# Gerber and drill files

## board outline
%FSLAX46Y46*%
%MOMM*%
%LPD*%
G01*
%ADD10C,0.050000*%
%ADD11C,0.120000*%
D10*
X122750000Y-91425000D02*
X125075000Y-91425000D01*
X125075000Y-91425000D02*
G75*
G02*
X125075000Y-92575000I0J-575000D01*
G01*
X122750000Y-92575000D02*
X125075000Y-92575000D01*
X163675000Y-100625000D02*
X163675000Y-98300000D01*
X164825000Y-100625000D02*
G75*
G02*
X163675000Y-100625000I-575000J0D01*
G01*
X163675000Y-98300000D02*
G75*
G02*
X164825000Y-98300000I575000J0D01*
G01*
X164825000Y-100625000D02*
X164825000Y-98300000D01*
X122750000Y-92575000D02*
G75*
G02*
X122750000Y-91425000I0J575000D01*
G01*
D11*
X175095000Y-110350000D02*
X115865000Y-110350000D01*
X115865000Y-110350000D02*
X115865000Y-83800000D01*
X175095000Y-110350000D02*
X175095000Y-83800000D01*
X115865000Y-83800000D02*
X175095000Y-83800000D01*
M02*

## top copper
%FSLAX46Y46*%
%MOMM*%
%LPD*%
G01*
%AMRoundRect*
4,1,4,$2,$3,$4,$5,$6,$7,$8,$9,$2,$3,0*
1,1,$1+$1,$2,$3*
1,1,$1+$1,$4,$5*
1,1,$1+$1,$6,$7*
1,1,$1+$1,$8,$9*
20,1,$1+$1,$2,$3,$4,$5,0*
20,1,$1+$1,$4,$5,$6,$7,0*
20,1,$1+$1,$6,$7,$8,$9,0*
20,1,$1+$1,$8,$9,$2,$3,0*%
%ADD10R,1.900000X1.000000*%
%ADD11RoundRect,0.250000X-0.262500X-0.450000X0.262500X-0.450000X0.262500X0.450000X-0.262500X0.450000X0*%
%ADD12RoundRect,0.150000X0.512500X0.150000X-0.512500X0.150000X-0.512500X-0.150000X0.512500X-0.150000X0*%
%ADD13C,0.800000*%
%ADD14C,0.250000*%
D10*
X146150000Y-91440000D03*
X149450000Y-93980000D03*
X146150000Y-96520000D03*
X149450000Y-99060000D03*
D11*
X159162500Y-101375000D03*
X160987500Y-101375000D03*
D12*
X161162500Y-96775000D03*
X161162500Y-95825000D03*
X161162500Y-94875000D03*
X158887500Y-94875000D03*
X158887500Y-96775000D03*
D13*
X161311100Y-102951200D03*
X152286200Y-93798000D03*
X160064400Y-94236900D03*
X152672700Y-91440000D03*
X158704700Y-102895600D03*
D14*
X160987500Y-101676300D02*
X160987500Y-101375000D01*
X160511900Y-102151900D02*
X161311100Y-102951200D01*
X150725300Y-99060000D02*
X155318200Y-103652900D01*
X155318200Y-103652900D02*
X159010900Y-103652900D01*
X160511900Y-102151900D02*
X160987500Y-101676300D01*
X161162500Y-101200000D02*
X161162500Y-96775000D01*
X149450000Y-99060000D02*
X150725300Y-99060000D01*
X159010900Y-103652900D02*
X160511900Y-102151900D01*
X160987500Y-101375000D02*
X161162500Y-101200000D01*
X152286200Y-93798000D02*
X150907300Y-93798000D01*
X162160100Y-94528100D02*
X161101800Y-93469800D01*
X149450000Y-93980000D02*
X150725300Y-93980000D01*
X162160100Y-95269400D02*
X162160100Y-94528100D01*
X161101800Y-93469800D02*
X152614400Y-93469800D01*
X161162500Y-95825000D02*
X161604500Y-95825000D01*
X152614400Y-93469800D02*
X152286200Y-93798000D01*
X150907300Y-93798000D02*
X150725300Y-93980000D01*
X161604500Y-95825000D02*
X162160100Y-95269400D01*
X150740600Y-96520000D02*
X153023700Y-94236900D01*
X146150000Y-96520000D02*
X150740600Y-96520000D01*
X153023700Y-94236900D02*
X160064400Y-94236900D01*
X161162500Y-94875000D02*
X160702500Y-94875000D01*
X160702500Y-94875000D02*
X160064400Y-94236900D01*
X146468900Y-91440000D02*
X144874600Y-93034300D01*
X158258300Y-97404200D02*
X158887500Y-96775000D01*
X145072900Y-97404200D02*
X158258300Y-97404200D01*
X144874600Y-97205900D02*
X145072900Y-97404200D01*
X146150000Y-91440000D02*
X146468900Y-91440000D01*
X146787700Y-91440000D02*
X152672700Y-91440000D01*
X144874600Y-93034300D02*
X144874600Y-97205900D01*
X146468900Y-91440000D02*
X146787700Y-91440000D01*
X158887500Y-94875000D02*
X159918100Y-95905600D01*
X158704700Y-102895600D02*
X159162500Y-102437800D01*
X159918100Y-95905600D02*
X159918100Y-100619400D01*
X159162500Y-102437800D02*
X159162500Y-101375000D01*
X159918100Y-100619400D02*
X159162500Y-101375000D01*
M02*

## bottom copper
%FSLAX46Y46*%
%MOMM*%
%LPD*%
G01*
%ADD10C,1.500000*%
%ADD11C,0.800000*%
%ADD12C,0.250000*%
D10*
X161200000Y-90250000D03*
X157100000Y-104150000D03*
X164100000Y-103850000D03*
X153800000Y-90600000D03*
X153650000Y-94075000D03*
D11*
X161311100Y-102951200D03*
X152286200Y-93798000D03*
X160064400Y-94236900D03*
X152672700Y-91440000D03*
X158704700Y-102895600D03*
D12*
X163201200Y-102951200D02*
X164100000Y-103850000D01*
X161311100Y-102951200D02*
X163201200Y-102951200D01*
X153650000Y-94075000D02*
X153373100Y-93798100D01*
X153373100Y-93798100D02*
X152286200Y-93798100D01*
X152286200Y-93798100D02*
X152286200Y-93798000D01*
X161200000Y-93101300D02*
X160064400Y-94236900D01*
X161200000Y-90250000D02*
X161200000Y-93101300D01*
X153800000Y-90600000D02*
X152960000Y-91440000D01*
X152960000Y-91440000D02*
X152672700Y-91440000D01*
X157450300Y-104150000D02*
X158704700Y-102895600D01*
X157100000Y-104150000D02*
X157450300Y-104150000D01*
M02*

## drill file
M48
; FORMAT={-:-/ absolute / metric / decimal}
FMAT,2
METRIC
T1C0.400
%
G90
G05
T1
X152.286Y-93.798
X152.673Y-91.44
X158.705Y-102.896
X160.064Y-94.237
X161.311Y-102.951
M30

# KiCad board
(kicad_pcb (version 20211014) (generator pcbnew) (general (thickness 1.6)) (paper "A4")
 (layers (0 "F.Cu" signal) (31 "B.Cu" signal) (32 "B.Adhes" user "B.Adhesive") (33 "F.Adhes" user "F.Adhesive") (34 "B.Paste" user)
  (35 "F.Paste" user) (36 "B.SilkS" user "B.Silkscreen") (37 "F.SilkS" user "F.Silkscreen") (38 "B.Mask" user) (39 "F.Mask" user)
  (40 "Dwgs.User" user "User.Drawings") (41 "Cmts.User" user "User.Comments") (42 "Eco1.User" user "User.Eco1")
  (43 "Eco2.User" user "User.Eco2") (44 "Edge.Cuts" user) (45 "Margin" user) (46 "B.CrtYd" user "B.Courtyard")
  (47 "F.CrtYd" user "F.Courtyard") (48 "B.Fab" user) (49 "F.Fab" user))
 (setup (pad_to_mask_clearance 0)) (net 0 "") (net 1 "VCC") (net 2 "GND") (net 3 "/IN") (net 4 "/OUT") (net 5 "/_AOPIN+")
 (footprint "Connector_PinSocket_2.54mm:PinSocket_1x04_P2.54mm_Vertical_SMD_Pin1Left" (layer "F.Cu") (at 147.8 95.25)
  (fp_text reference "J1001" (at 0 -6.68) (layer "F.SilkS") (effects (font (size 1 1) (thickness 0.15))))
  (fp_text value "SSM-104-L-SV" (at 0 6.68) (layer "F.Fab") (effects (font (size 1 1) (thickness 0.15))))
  (pad "1" smd rect locked (at -1.65 -3.81) (size 1.9 1) (layers "F.Cu" "F.Paste" "F.Mask") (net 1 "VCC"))
  (pad "2" smd rect locked (at 1.65 -1.27) (size 1.9 1) (layers "F.Cu" "F.Paste" "F.Mask") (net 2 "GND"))
  (pad "3" smd rect locked (at -1.65 1.27) (size 1.9 1) (layers "F.Cu" "F.Paste" "F.Mask") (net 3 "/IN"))
  (pad "4" smd rect locked (at 1.65 3.81) (size 1.9 1) (layers "F.Cu" "F.Paste" "F.Mask") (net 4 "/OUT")))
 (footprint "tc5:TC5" (layer "F.Cu") (at 135.3 97.9)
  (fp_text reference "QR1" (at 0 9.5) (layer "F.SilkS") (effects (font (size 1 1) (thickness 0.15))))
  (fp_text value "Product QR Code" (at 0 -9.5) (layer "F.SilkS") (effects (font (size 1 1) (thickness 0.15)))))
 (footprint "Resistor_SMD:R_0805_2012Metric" (layer "F.Cu") (at 160.075 101.375)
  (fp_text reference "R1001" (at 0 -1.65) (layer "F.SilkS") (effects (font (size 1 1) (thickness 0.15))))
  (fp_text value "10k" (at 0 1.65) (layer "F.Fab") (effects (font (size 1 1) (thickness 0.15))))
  (pad "1" smd roundrect locked (at -0.9125 0) (size 1.025 1.4) (layers "F.Cu" "F.Paste" "F.Mask") (roundrect_rratio 0.243902)
   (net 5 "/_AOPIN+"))
  (pad "2" smd roundrect locked (at 0.9125 0) (size 1.025 1.4) (layers "F.Cu" "F.Paste" "F.Mask") (roundrect_rratio 0.243902) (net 4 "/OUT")))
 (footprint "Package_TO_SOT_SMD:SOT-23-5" (layer "F.Cu") (at 160.025 95.825 180)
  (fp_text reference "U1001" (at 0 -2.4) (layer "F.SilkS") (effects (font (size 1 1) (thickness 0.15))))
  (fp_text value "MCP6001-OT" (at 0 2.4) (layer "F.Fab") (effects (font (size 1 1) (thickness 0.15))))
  (pad "1" smd roundrect locked (at -1.1375 -0.95 180) (size 1.325 0.6) (layers "F.Cu" "F.Paste" "F.Mask") (roundrect_rratio 0.25)
   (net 4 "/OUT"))
  (pad "2" smd roundrect locked (at -1.1375 0 180) (size 1.325 0.6) (layers "F.Cu" "F.Paste" "F.Mask") (roundrect_rratio 0.25) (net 2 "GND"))
  (pad "3" smd roundrect locked (at -1.1375 0.95 180) (size 1.325 0.6) (layers "F.Cu" "F.Paste" "F.Mask") (roundrect_rratio 0.25)
   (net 3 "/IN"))
  (pad "4" smd roundrect locked (at 1.1375 0.95 180) (size 1.325 0.6) (layers "F.Cu" "F.Paste" "F.Mask") (roundrect_rratio 0.25)
   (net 5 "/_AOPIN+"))
  (pad "5" smd roundrect locked (at 1.1375 -0.95 180) (size 1.325 0.6) (layers "F.Cu" "F.Paste" "F.Mask") (roundrect_rratio 0.25)
   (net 1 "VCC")))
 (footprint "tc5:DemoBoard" (layer "F.Cu") (at 127.325 91.1)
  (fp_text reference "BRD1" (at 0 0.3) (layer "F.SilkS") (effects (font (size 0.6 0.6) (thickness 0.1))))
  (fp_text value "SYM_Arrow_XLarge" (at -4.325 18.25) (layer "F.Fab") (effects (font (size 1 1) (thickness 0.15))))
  (fp_line (start 47.77 19.25) (end -11.46 19.25) (layer "Edge.Cuts") (width 0.12))
  (fp_line (start -11.46 19.25) (end -11.46 -7.3) (layer "Edge.Cuts") (width 0.12))
  (fp_line (start 47.77 19.25) (end 47.77 -7.3) (layer "Edge.Cuts") (width 0.12))
  (fp_line (start -11.46 -7.3) (end 47.77 -7.3) (layer "Edge.Cuts") (width 0.12)))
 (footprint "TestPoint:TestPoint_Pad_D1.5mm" (layer "B.Cu") (at 161.2 90.25)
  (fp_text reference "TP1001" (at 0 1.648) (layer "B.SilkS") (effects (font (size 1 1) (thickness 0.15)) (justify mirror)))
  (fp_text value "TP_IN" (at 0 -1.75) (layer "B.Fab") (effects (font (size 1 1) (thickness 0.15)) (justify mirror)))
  (pad "1" smd circle locked (at 0 0) (size 1.5 1.5) (layers "B.Cu" "B.Mask") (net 3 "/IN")))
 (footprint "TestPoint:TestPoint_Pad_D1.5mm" (layer "B.Cu") (at 157.1 104.15)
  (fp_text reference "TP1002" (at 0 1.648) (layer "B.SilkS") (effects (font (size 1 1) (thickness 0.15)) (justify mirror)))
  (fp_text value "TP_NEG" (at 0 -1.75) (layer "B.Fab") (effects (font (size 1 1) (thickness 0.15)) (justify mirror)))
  (pad "1" smd circle locked (at 0 0) (size 1.5 1.5) (layers "B.Cu" "B.Mask") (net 5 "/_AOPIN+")))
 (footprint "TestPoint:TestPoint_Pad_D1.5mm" (layer "B.Cu") (at 164.1 103.85 180)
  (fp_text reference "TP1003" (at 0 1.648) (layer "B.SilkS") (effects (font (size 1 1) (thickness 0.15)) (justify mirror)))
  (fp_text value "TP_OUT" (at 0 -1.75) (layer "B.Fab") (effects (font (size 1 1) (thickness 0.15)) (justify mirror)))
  (pad "1" smd circle locked (at 0 0 180) (size 1.5 1.5) (layers "B.Cu" "B.Mask") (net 4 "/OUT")))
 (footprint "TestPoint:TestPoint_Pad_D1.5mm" (layer "B.Cu") (at 153.8 90.6)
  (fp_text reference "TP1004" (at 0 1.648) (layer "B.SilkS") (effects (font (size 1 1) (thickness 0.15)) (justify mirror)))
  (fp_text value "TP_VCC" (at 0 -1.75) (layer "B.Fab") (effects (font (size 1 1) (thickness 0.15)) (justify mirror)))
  (pad "1" smd circle locked (at 0 0) (size 1.5 1.5) (layers "B.Cu" "B.Mask") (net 1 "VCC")))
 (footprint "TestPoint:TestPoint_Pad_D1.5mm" (layer "B.Cu") (at 153.65 94.075)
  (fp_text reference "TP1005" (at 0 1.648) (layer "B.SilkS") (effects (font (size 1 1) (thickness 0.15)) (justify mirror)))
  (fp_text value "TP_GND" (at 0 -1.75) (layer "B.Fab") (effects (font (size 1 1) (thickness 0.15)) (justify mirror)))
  (pad "1" smd circle locked (at 0 0) (size 1.5 1.5) (layers "B.Cu" "B.Mask") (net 2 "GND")))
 (gr_line (start 122.75 91.425) (end 125.075 91.425) (layer "Edge.Cuts") (width 0.05))
 (gr_arc (start 125.075 91.425) (mid 125.65 92) (end 125.075 92.575) (layer "Edge.Cuts") (width 0.05))
 (gr_line (start 122.75 92.575) (end 125.075 92.575) (layer "Edge.Cuts") (width 0.05))
 (gr_line (start 163.675 100.625) (end 163.675 98.3) (layer "Edge.Cuts") (width 0.05))
 (gr_arc (start 164.825 100.625) (mid 164.25 101.2) (end 163.675 100.625) (layer "Edge.Cuts") (width 0.05))
 (gr_arc (start 163.675 98.3) (mid 164.25 97.725) (end 164.825 98.3) (layer "Edge.Cuts") (width 0.05))
 (gr_line (start 164.825 100.625) (end 164.825 98.3) (layer "Edge.Cuts") (width 0.05))
 (gr_arc (start 122.75 92.575) (mid 122.175 92) (end 122.75 91.425) (layer "Edge.Cuts") (width 0.05))
 (segment (start 160.9875 101.6763) (end 160.9875 101.375) (width 0.25) (layer "F.Cu") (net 4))
 (segment (start 160.5119 102.1519) (end 161.3111 102.9512) (width 0.25) (layer "F.Cu") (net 4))
 (segment (start 150.7253 99.06) (end 155.3182 103.6529) (width 0.25) (layer "F.Cu") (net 4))
 (segment (start 155.3182 103.6529) (end 159.0109 103.6529) (width 0.25) (layer "F.Cu") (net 4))
 (segment (start 160.5119 102.1519) (end 160.9875 101.6763) (width 0.25) (layer "F.Cu") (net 4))
 (segment (start 161.1625 101.2) (end 161.1625 96.775) (width 0.25) (layer "F.Cu") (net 4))
 (segment (start 149.45 99.06) (end 150.7253 99.06) (width 0.25) (layer "F.Cu") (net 4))
 (segment (start 159.0109 103.6529) (end 160.5119 102.1519) (width 0.25) (layer "F.Cu") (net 4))
 (segment (start 160.9875 101.375) (end 161.1625 101.2) (width 0.25) (layer "F.Cu") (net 4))
 (via (at 161.3111 102.9512) (size 0.8) (drill 0.4) (layers "F.Cu" "B.Cu") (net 4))
 (segment (start 163.2012 102.9512) (end 164.1 103.85) (width 0.25) (layer "B.Cu") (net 4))
 (segment (start 161.3111 102.9512) (end 163.2012 102.9512) (width 0.25) (layer "B.Cu") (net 4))
 (segment (start 152.2862 93.798) (end 150.9073 93.798) (width 0.25) (layer "F.Cu") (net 2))
 (segment (start 162.1601 94.5281) (end 161.1018 93.4698) (width 0.25) (layer "F.Cu") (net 2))
 (segment (start 149.45 93.98) (end 150.7253 93.98) (width 0.25) (layer "F.Cu") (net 2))
 (segment (start 162.1601 95.2694) (end 162.1601 94.5281) (width 0.25) (layer "F.Cu") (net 2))
 (segment (start 161.1018 93.4698) (end 152.6144 93.4698) (width 0.25) (layer "F.Cu") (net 2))
 (segment (start 161.1625 95.825) (end 161.6045 95.825) (width 0.25) (layer "F.Cu") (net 2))
 (segment (start 152.6144 93.4698) (end 152.2862 93.798) (width 0.25) (layer "F.Cu") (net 2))
 (segment (start 150.9073 93.798) (end 150.7253 93.98) (width 0.25) (layer "F.Cu") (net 2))
 (segment (start 161.6045 95.825) (end 162.1601 95.2694) (width 0.25) (layer "F.Cu") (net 2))
 (via (at 152.2862 93.798) (size 0.8) (drill 0.4) (layers "F.Cu" "B.Cu") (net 2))
 (segment (start 153.65 94.075) (end 153.3731 93.7981) (width 0.25) (layer "B.Cu") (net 2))
 (segment (start 153.3731 93.7981) (end 152.2862 93.7981) (width 0.25) (layer "B.Cu") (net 2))
 (segment (start 152.2862 93.7981) (end 152.2862 93.798) (width 0.25) (layer "B.Cu") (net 2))
 (segment (start 150.7406 96.52) (end 153.0237 94.2369) (width 0.25) (layer "F.Cu") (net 3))
 (segment (start 146.15 96.52) (end 150.7406 96.52) (width 0.25) (layer "F.Cu") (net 3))
 (segment (start 153.0237 94.2369) (end 160.0644 94.2369) (width 0.25) (layer "F.Cu") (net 3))
 (segment (start 161.1625 94.875) (end 160.7025 94.875) (width 0.25) (layer "F.Cu") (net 3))
 (segment (start 160.7025 94.875) (end 160.0644 94.2369) (width 0.25) (layer "F.Cu") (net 3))
 (via (at 160.0644 94.2369) (size 0.8) (drill 0.4) (layers "F.Cu" "B.Cu") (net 3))
 (segment (start 161.2 93.1013) (end 160.0644 94.2369) (width 0.25) (layer "B.Cu") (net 3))
 (segment (start 161.2 90.25) (end 161.2 93.1013) (width 0.25) (layer "B.Cu") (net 3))
 (segment (start 146.4689 91.44) (end 144.8746 93.0343) (width 0.25) (layer "F.Cu") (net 1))
 (segment (start 158.2583 97.4042) (end 158.8875 96.775) (width 0.25) (layer "F.Cu") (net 1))
 (segment (start 145.0729 97.4042) (end 158.2583 97.4042) (width 0.25) (layer "F.Cu") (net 1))
 (segment (start 144.8746 97.2059) (end 145.0729 97.4042) (width 0.25) (layer "F.Cu") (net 1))
 (segment (start 146.15 91.44) (end 146.4689 91.44) (width 0.25) (layer "F.Cu") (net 1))
 (segment (start 146.7877 91.44) (end 152.6727 91.44) (width 0.25) (layer "F.Cu") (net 1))
 (segment (start 144.8746 93.0343) (end 144.8746 97.2059) (width 0.25) (layer "F.Cu") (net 1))
 (segment (start 146.4689 91.44) (end 146.7877 91.44) (width 0.25) (layer "F.Cu") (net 1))
 (via (at 152.6727 91.44) (size 0.8) (drill 0.4) (layers "F.Cu" "B.Cu") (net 1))
 (segment (start 153.8 90.6) (end 152.96 91.44) (width 0.25) (layer "B.Cu") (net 1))
 (segment (start 152.96 91.44) (end 152.6727 91.44) (width 0.25) (layer "B.Cu") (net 1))
 (segment (start 158.8875 94.875) (end 159.9181 95.9056) (width 0.25) (layer "F.Cu") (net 5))
 (segment (start 158.7047 102.8956) (end 159.1625 102.4378) (width 0.25) (layer "F.Cu") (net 5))
 (segment (start 159.9181 95.9056) (end 159.9181 100.6194) (width 0.25) (layer "F.Cu") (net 5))
 (segment (start 159.1625 102.4378) (end 159.1625 101.375) (width 0.25) (layer "F.Cu") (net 5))
 (segment (start 159.9181 100.6194) (end 159.1625 101.375) (width 0.25) (layer "F.Cu") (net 5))
 (via (at 158.7047 102.8956) (size 0.8) (drill 0.4) (layers "F.Cu" "B.Cu") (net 5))
 (segment (start 157.4503 104.15) (end 158.7047 102.8956) (width 0.25) (layer "B.Cu") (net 5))
 (segment (start 157.1 104.15) (end 157.4503 104.15) (width 0.25) (layer "B.Cu") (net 5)))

